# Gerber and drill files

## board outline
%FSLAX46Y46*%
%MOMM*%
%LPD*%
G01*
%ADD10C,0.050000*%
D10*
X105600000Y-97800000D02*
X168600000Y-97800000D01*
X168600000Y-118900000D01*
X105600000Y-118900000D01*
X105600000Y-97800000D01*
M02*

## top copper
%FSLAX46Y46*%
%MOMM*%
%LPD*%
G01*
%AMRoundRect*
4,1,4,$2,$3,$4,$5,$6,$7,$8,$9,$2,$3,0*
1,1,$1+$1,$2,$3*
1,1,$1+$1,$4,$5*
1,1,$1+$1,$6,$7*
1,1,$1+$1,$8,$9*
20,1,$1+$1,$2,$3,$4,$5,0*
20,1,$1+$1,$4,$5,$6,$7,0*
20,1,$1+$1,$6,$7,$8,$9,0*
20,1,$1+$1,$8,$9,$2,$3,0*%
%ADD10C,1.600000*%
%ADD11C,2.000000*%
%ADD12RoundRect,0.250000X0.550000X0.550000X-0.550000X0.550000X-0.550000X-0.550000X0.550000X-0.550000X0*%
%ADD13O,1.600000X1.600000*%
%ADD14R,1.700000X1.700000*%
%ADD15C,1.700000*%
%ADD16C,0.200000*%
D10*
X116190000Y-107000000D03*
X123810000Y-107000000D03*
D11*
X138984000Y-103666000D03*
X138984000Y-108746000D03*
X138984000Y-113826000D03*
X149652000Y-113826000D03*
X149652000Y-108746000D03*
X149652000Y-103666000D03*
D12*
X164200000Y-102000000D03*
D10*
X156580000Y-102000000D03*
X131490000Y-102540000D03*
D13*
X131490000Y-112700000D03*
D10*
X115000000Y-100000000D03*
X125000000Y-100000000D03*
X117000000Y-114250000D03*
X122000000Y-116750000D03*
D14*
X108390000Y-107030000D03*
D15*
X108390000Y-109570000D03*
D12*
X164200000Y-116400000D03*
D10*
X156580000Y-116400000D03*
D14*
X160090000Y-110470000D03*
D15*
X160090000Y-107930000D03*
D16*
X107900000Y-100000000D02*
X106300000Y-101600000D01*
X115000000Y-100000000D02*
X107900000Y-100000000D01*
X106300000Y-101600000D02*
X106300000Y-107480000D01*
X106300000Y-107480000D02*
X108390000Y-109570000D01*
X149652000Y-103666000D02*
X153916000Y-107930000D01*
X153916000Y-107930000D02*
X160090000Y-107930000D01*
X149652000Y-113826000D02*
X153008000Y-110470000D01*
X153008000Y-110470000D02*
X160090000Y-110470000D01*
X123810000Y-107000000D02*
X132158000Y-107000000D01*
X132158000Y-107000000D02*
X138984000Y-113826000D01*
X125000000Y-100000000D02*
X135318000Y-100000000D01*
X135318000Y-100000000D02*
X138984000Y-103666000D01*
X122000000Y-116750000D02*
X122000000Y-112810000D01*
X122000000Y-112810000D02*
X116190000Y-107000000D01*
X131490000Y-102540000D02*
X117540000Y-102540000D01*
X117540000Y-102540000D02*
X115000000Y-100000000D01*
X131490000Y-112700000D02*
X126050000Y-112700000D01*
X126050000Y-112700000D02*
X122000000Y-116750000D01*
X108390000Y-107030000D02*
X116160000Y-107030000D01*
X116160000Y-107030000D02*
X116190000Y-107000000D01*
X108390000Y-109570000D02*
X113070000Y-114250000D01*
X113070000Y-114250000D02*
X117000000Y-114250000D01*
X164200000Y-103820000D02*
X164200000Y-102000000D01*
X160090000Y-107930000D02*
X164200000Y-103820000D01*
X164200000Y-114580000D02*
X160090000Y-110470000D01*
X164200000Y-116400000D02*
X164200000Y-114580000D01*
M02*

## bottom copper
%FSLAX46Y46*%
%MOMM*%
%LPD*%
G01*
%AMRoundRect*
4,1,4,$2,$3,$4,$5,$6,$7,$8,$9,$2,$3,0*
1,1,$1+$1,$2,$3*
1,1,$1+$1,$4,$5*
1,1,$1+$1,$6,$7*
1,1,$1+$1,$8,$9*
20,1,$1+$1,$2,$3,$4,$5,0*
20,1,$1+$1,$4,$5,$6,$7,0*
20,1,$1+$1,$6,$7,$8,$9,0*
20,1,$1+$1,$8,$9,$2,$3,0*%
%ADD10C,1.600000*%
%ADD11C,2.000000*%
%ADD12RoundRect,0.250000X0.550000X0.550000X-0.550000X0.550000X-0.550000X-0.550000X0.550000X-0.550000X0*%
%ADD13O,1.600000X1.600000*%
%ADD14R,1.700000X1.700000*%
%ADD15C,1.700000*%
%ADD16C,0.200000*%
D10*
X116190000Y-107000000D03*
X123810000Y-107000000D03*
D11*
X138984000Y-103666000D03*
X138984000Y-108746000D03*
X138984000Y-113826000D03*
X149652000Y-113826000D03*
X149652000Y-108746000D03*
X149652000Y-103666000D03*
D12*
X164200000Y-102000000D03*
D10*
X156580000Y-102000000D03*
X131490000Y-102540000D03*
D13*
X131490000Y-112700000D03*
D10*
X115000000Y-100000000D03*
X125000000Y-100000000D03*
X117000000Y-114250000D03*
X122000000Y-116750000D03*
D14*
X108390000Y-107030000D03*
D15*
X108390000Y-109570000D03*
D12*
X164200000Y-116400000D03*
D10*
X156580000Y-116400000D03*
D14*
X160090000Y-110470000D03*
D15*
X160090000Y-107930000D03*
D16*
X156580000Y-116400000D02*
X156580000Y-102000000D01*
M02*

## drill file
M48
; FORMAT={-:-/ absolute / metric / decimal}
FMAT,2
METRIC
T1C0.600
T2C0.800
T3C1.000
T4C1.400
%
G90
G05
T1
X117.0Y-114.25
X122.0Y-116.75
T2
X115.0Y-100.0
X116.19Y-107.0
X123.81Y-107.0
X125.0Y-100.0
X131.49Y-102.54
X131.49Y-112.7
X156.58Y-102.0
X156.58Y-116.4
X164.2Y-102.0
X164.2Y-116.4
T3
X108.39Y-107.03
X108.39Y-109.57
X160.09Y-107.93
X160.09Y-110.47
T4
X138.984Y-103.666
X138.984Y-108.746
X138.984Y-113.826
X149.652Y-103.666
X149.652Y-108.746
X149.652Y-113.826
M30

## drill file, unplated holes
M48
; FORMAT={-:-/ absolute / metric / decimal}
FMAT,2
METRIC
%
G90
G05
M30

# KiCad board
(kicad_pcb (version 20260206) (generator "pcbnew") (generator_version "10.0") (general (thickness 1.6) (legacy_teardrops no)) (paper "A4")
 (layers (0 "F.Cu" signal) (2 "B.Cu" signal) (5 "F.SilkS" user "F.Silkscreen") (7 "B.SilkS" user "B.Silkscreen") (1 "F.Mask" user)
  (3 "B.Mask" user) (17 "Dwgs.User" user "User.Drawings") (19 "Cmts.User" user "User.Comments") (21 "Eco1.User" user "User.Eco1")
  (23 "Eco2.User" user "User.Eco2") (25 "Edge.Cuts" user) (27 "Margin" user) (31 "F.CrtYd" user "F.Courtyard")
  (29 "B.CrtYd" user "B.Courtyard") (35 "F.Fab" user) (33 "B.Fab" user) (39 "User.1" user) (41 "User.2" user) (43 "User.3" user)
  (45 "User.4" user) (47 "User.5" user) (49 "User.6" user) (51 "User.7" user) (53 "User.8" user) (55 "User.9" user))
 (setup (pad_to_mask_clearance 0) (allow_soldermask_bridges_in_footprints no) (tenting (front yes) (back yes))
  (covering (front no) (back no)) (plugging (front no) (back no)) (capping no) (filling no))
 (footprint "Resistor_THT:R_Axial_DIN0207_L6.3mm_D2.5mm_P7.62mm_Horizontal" (layer "F.Cu") (at 116.19 107)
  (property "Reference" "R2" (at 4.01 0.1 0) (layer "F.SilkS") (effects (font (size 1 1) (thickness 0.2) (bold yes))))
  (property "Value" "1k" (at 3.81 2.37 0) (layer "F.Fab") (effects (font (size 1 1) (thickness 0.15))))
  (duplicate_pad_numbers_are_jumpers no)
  (pad "1" thru_hole circle (at 0 0) (size 1.6 1.6) (drill 0.8) (layers "*.Cu" "*.Mask") (remove_unused_layers no) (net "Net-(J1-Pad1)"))
  (pad "2" thru_hole circle (at 7.62 0) (size 1.6 1.6) (drill 0.8) (layers "*.Cu" "*.Mask") (remove_unused_layers no) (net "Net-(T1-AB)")))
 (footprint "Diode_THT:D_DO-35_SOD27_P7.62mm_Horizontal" (layer "F.Cu") (at 164.2 102 180)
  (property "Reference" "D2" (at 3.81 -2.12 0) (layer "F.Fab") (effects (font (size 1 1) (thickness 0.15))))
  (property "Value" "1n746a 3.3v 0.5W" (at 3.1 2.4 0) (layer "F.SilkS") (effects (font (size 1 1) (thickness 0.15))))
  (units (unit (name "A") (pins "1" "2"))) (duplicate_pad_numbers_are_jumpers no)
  (pad "1" thru_hole roundrect (at 0 0 180) (size 1.6 1.6) (drill 0.8) (layers "*.Cu" "*.Mask") (remove_unused_layers no)
   (roundrect_rratio 0.15625) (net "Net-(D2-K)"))
  (pad "2" thru_hole circle (at 7.62 0 180) (size 1.6 1.6) (drill 0.8) (layers "*.Cu" "*.Mask") (remove_unused_layers no) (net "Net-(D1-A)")))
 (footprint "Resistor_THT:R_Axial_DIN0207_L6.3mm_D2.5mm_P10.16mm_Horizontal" (layer "F.Cu") (at 131.49 102.54 -90)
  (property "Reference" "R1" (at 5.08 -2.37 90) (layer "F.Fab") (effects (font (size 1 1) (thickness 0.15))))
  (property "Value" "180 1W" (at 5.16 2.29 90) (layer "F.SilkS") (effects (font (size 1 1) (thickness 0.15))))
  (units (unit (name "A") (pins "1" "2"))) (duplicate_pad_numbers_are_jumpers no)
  (pad "1" thru_hole circle (at 0 0 270) (size 1.6 1.6) (drill 0.8) (layers "*.Cu" "*.Mask") (remove_unused_layers no) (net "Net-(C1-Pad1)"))
  (pad "2" thru_hole oval (at 10.16 0 270) (size 1.6 1.6) (drill 0.8) (layers "*.Cu" "*.Mask") (remove_unused_layers no)
   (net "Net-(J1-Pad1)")))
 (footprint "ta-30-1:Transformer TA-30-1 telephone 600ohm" (layer "F.Cu") (at 138.984 108.746)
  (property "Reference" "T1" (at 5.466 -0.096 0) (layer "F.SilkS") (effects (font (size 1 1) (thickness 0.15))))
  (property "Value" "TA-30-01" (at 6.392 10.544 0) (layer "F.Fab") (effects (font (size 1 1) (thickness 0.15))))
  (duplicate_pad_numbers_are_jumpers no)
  (pad "1" thru_hole circle (at 0 -5.08) (size 2 2) (drill 1.4) (layers "*.Cu" "*.Mask") (remove_unused_layers no) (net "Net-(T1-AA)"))
  (pad "2" thru_hole circle (at 0 0) (size 2 2) (drill 1.4) (layers "*.Cu" "*.Mask") (remove_unused_layers no)
   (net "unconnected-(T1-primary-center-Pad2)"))
  (pad "3" thru_hole circle (at 0 5.08) (size 2 2) (drill 1.4) (layers "*.Cu" "*.Mask") (remove_unused_layers no) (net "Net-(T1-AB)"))
  (pad "4" thru_hole circle (at 10.668 5.08) (size 2 2) (drill 1.4) (layers "*.Cu" "*.Mask") (remove_unused_layers no) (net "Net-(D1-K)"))
  (pad "5" thru_hole circle (at 10.668 0) (size 2 2) (drill 1.4) (layers "*.Cu" "*.Mask") (remove_unused_layers no)
   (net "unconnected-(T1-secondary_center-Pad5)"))
  (pad "6" thru_hole circle (at 10.668 -5.08) (size 2 2) (drill 1.4) (layers "*.Cu" "*.Mask") (remove_unused_layers no) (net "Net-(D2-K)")))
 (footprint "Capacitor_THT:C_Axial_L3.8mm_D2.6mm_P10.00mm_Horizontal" (layer "F.Cu") (at 115 100)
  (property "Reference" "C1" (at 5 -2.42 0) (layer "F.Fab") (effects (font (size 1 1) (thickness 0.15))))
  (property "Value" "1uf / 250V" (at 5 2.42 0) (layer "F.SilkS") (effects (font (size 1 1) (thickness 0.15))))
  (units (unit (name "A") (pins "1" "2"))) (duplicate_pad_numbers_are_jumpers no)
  (pad "1" thru_hole circle (at 0 0) (size 1.6 1.6) (drill 0.8) (layers "*.Cu" "*.Mask") (remove_unused_layers no) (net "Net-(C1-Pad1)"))
  (pad "2" thru_hole circle (at 10 0) (size 1.6 1.6) (drill 0.8) (layers "*.Cu" "*.Mask") (remove_unused_layers no) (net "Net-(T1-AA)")))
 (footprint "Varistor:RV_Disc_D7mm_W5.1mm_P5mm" (layer "F.Cu") (at 117 114.25)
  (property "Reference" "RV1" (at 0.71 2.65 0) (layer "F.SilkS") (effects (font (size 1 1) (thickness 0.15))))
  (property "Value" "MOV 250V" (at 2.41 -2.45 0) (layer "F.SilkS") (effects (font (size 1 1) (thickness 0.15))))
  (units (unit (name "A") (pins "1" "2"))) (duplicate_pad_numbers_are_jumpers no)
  (pad "1" thru_hole circle (at 0 0) (size 1.6 1.6) (drill 0.6) (layers "*.Cu" "*.Mask") (remove_unused_layers no) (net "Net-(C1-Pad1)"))
  (pad "2" thru_hole circle (at 5 2.5) (size 1.6 1.6) (drill 0.6) (layers "*.Cu" "*.Mask") (remove_unused_layers no) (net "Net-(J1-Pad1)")))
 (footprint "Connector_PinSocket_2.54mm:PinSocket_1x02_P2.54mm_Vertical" (layer "F.Cu") (at 108.39 107.03)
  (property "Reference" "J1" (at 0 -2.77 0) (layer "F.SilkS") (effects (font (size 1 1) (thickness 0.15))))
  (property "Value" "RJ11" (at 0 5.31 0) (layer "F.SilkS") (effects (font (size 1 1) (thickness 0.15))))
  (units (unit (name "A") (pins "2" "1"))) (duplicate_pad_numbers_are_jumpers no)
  (pad "1" thru_hole rect (at 0 0) (size 1.7 1.7) (drill 1) (layers "*.Cu" "*.Mask") (remove_unused_layers no) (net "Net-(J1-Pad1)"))
  (pad "2" thru_hole circle (at 0 2.54) (size 1.7 1.7) (drill 1) (layers "*.Cu" "*.Mask") (remove_unused_layers no) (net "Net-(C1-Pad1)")))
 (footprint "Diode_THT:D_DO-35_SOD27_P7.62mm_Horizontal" (layer "F.Cu") (at 164.2 116.4 180)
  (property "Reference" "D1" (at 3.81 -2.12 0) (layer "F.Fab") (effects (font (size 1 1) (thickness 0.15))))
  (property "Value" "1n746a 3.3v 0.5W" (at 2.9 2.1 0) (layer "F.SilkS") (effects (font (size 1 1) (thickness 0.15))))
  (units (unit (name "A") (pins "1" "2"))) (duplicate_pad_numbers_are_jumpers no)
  (pad "1" thru_hole roundrect (at 0 0 180) (size 1.6 1.6) (drill 0.8) (layers "*.Cu" "*.Mask") (remove_unused_layers no)
   (roundrect_rratio 0.15625) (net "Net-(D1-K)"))
  (pad "2" thru_hole circle (at 7.62 0 180) (size 1.6 1.6) (drill 0.8) (layers "*.Cu" "*.Mask") (remove_unused_layers no) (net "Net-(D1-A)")))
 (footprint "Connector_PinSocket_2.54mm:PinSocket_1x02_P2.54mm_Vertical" (layer "F.Cu") (at 160.09 110.47 180)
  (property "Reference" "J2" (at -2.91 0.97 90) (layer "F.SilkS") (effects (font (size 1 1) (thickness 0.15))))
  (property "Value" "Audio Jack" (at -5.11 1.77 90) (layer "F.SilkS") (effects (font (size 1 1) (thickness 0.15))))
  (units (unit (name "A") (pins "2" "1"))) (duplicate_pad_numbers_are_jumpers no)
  (pad "1" thru_hole rect (at 0 0 180) (size 1.7 1.7) (drill 1) (layers "*.Cu" "*.Mask") (remove_unused_layers no) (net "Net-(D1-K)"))
  (pad "2" thru_hole circle (at 0 2.54 180) (size 1.7 1.7) (drill 1) (layers "*.Cu" "*.Mask") (remove_unused_layers no) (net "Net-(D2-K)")))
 (gr_rect (start 105.6 97.8) (end 168.6 118.9) (stroke (width 0.05) (type default)) (fill no) (layer "Edge.Cuts"))
 (segment (start 116.16 107.03) (end 116.19 107) (width 0.2) (layer "F.Cu") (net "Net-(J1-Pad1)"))
 (segment (start 108.39 107.03) (end 116.16 107.03) (width 0.2) (layer "F.Cu") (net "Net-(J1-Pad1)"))
 (segment (start 122 116.75) (end 122 112.81) (width 0.2) (layer "F.Cu") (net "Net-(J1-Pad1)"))
 (segment (start 122 112.81) (end 116.19 107) (width 0.2) (layer "F.Cu") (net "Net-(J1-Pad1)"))
 (segment (start 131.49 112.7) (end 126.05 112.7) (width 0.2) (layer "F.Cu") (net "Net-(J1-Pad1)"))
 (segment (start 126.05 112.7) (end 122 116.75) (width 0.2) (layer "F.Cu") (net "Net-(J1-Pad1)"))
 (segment (start 123.81 107) (end 132.158 107) (width 0.2) (layer "F.Cu") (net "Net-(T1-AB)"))
 (segment (start 132.158 107) (end 138.984 113.826) (width 0.2) (layer "F.Cu") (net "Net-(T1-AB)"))
 (segment (start 149.652 103.666) (end 153.916 107.93) (width 0.2) (layer "F.Cu") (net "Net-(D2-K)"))
 (segment (start 164.2 103.82) (end 164.2 102) (width 0.2) (layer "F.Cu") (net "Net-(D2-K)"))
 (segment (start 160.09 107.93) (end 164.2 103.82) (width 0.2) (layer "F.Cu") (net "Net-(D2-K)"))
 (segment (start 153.916 107.93) (end 160.09 107.93) (width 0.2) (layer "F.Cu") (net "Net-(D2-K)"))
 (segment (start 156.58 116.4) (end 156.58 102) (width 0.2) (layer "B.Cu") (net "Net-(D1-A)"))
 (segment (start 107.9 100) (end 106.3 101.6) (width 0.2) (layer "F.Cu") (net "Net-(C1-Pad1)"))
 (segment (start 131.49 102.54) (end 117.54 102.54) (width 0.2) (layer "F.Cu") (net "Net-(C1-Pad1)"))
 (segment (start 106.3 101.6) (end 106.3 107.48) (width 0.2) (layer "F.Cu") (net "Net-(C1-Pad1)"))
 (segment (start 106.3 107.48) (end 108.39 109.57) (width 0.2) (layer "F.Cu") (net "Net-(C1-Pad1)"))
 (segment (start 113.07 114.25) (end 117 114.25) (width 0.2) (layer "F.Cu") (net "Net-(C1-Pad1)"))
 (segment (start 117.54 102.54) (end 115 100) (width 0.2) (layer "F.Cu") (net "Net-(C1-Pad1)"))
 (segment (start 115 100) (end 107.9 100) (width 0.2) (layer "F.Cu") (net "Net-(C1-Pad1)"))
 (segment (start 108.39 109.57) (end 113.07 114.25) (width 0.2) (layer "F.Cu") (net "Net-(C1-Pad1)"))
 (segment (start 125 100) (end 135.318 100) (width 0.2) (layer "F.Cu") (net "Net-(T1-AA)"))
 (segment (start 135.318 100) (end 138.984 103.666) (width 0.2) (layer "F.Cu") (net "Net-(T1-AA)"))
 (segment (start 149.652 113.826) (end 153.008 110.47) (width 0.2) (layer "F.Cu") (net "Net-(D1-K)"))
 (segment (start 164.2 114.58) (end 160.09 110.47) (width 0.2) (layer "F.Cu") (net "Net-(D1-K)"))
 (segment (start 164.2 116.4) (end 164.2 114.58) (width 0.2) (layer "F.Cu") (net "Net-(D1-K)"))
 (segment (start 153.008 110.47) (end 160.09 110.47) (width 0.2) (layer "F.Cu") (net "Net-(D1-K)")))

